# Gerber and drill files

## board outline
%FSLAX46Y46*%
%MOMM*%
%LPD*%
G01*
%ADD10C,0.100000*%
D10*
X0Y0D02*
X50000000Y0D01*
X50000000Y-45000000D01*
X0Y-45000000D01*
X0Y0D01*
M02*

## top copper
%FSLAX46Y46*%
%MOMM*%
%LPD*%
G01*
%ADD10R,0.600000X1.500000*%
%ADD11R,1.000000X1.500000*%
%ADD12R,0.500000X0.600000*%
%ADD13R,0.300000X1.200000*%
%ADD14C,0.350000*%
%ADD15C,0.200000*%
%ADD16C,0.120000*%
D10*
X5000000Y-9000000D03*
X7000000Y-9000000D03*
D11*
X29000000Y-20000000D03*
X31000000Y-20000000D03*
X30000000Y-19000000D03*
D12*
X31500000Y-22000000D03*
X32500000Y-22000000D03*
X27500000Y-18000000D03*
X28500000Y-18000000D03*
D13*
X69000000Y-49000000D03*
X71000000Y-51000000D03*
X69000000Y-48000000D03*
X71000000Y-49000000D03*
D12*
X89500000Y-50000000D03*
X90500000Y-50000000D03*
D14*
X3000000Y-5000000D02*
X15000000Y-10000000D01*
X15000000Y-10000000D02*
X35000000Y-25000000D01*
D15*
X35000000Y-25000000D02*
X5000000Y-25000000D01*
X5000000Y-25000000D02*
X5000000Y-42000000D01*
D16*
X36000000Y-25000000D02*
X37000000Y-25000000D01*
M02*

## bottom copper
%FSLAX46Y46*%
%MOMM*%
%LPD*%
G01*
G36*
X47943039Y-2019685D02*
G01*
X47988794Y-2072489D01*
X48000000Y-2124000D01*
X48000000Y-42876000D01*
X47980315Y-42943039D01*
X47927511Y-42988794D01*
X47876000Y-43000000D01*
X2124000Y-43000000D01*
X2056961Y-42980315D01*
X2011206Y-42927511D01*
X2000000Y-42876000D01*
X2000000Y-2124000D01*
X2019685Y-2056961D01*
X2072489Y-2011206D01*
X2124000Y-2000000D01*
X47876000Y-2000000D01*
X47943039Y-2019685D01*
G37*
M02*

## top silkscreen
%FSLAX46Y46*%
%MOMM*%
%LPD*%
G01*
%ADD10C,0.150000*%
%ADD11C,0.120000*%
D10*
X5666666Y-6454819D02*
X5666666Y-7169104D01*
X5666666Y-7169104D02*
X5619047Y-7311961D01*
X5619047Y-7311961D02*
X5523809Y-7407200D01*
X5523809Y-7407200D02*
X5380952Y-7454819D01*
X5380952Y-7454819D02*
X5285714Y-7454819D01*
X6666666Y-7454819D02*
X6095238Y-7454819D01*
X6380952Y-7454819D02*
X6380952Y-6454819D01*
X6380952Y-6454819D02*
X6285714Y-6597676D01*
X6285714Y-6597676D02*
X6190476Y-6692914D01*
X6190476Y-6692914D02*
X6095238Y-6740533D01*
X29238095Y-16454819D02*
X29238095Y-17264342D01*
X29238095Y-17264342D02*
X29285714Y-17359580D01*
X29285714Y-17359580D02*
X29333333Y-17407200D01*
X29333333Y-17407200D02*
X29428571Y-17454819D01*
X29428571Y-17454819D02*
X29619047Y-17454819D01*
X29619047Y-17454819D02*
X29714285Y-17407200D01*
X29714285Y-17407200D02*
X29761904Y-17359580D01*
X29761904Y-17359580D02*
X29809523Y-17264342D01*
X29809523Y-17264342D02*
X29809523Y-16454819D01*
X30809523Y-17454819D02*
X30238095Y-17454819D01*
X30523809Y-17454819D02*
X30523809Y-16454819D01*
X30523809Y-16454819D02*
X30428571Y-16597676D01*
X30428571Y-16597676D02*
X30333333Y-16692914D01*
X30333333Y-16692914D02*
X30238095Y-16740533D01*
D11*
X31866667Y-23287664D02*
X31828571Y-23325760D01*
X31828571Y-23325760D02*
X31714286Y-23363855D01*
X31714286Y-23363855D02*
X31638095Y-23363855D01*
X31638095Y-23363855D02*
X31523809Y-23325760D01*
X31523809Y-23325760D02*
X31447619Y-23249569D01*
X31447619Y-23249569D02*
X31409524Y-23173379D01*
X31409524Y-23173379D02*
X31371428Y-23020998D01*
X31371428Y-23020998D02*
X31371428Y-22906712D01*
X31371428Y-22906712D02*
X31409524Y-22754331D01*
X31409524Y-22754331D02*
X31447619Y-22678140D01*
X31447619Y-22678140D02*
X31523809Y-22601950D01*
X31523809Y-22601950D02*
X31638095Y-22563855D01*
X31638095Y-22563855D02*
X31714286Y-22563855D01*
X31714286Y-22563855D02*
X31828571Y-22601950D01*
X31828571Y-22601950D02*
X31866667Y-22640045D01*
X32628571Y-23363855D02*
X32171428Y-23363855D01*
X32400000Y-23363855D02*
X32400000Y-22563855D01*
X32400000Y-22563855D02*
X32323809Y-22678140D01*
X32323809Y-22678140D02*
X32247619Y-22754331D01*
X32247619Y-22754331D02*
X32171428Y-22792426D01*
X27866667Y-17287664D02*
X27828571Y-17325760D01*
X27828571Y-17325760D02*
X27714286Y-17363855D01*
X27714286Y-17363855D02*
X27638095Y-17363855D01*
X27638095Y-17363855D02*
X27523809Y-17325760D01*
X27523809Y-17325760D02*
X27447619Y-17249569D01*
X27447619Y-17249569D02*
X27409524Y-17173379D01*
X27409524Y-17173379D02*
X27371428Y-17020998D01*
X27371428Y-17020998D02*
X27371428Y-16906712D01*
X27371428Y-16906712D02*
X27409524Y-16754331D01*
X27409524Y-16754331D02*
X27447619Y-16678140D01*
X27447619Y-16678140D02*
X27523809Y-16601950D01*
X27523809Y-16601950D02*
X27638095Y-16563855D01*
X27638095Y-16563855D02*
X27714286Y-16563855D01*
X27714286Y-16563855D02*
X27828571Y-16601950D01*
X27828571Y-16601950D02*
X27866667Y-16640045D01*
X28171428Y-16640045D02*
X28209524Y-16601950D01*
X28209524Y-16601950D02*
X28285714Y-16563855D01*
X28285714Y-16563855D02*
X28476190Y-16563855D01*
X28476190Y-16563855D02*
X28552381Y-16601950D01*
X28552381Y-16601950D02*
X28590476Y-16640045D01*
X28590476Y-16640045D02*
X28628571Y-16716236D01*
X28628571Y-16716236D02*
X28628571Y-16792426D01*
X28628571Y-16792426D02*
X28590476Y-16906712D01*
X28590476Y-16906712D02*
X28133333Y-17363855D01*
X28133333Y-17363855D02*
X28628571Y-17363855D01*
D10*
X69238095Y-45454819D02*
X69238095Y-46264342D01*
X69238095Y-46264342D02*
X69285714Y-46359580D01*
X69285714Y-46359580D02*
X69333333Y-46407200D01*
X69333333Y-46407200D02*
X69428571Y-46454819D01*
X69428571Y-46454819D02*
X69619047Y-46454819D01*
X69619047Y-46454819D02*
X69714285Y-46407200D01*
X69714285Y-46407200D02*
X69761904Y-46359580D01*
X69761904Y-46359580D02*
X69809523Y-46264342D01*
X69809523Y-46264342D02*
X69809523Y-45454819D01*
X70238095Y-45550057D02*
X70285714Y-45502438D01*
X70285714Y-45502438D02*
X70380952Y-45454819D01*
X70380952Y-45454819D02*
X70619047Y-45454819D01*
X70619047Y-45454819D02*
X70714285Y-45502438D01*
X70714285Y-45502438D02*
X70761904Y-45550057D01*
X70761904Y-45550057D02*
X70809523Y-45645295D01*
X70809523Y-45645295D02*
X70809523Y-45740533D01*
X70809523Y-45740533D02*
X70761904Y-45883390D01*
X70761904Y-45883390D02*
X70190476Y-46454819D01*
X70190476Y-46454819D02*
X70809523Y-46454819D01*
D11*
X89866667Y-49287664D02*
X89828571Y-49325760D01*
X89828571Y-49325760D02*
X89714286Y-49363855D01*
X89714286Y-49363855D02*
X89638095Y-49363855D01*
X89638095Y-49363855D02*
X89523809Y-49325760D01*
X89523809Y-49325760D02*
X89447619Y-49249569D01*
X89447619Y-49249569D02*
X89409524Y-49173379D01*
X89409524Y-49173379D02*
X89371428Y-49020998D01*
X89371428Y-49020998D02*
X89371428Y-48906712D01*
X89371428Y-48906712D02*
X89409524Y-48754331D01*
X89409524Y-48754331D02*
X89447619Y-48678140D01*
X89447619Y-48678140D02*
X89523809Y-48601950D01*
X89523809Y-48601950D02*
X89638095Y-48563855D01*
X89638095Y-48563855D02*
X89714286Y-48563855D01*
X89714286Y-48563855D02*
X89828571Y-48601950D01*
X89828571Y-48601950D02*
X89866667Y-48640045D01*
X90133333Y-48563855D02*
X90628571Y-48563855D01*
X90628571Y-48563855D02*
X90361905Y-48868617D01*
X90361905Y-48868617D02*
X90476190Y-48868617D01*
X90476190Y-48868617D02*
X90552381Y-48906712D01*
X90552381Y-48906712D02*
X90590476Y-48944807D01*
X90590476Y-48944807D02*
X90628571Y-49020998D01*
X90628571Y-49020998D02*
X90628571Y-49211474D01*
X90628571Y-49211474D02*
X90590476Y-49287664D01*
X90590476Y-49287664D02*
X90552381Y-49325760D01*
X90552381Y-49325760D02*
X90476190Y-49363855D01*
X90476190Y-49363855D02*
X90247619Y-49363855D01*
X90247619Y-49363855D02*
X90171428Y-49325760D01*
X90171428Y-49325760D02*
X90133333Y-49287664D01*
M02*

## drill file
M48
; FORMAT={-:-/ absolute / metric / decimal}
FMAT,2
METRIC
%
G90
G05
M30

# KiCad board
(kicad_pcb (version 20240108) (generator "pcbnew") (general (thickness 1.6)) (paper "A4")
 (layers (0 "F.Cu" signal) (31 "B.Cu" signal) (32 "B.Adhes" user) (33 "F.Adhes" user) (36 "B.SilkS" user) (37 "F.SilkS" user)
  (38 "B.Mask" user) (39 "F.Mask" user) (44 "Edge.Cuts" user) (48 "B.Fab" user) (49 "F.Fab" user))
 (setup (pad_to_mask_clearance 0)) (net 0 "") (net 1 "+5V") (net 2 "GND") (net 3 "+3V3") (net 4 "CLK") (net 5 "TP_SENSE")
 (gr_rect (start 0 0) (end 50 45) (layer "Edge.Cuts") (width 0.1))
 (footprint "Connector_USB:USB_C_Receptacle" (layer "F.Cu") (at 3 5 0)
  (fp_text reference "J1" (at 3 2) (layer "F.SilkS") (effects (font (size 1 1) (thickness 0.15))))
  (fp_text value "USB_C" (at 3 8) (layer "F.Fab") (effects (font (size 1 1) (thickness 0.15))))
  (pad "VBUS" smd rect (at 2 4) (size 0.6 1.5) (layers "F.Cu" "F.Paste" "F.Mask") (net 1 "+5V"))
  (pad "GND" smd rect (at 4 4) (size 0.6 1.5) (layers "F.Cu" "F.Paste" "F.Mask") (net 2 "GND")))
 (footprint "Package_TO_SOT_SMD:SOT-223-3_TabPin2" (layer "F.Cu") (at 15 10 0)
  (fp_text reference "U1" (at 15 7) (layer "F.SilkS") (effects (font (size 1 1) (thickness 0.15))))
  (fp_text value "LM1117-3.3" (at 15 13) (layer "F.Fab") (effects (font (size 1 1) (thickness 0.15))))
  (pad "1" smd rect (at 14 10) (size 1 1.5) (layers "F.Cu" "F.Paste" "F.Mask") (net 2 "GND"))
  (pad "2" smd rect (at 16 10) (size 1 1.5) (layers "F.Cu" "F.Paste" "F.Mask") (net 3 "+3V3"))
  (pad "3" smd rect (at 15 9) (size 1 1.5) (layers "F.Cu" "F.Paste" "F.Mask") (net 1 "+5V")))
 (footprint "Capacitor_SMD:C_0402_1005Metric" (layer "F.Cu") (at 16 11 0)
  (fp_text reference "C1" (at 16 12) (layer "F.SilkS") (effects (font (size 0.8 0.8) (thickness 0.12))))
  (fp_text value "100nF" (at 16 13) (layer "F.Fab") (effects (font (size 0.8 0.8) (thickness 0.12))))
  (pad "1" smd rect (at 15.5 11) (size 0.5 0.6) (layers "F.Cu" "F.Paste" "F.Mask") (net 3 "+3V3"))
  (pad "2" smd rect (at 16.5 11) (size 0.5 0.6) (layers "F.Cu" "F.Paste" "F.Mask") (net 2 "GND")))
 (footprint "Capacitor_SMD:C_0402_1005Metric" (layer "F.Cu") (at 14 9 0)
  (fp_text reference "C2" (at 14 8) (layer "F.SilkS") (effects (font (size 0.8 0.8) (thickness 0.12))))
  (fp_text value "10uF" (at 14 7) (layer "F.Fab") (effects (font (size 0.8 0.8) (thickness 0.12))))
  (pad "1" smd rect (at 13.5 9) (size 0.5 0.6) (layers "F.Cu" "F.Paste" "F.Mask") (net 1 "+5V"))
  (pad "2" smd rect (at 14.5 9) (size 0.5 0.6) (layers "F.Cu" "F.Paste" "F.Mask") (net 2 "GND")))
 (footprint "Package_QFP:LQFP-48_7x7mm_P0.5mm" (layer "F.Cu") (at 35 25 0)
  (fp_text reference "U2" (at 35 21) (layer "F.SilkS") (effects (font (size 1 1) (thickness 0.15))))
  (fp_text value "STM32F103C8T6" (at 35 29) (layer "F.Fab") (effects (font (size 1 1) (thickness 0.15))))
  (pad "8" smd rect (at 34 24) (size 0.3 1.2) (layers "F.Cu" "F.Paste" "F.Mask") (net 3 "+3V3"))
  (pad "23" smd rect (at 36 26) (size 0.3 1.2) (layers "F.Cu" "F.Paste" "F.Mask") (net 2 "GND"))
  (pad "5" smd rect (at 34 23) (size 0.3 1.2) (layers "F.Cu" "F.Paste" "F.Mask") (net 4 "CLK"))
  (pad "20" smd rect (at 36 24) (size 0.3 1.2) (layers "F.Cu" "F.Paste" "F.Mask") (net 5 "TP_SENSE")))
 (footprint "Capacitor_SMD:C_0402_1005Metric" (layer "F.Cu") (at 45 25 0)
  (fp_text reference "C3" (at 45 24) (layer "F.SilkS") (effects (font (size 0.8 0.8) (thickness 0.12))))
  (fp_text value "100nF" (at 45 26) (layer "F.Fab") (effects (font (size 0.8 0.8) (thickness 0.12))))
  (pad "1" smd rect (at 44.5 25) (size 0.5 0.6) (layers "F.Cu" "F.Paste" "F.Mask") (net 3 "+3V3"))
  (pad "2" smd rect (at 45.5 25) (size 0.5 0.6) (layers "F.Cu" "F.Paste" "F.Mask") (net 2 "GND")))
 (segment (start 3 5) (end 15 10) (width 0.35) (layer "F.Cu") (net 1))
 (segment (start 15 10) (end 35 25) (width 0.35) (layer "F.Cu") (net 3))
 (segment (start 35 25) (end 5 25) (width 0.2) (layer "F.Cu") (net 4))
 (segment (start 5 25) (end 5 42) (width 0.2) (layer "F.Cu") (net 4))
 (segment (start 36 25) (end 37 25) (width 0.12) (layer "F.Cu") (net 5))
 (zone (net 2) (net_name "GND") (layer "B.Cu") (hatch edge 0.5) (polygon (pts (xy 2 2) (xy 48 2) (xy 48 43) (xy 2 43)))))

